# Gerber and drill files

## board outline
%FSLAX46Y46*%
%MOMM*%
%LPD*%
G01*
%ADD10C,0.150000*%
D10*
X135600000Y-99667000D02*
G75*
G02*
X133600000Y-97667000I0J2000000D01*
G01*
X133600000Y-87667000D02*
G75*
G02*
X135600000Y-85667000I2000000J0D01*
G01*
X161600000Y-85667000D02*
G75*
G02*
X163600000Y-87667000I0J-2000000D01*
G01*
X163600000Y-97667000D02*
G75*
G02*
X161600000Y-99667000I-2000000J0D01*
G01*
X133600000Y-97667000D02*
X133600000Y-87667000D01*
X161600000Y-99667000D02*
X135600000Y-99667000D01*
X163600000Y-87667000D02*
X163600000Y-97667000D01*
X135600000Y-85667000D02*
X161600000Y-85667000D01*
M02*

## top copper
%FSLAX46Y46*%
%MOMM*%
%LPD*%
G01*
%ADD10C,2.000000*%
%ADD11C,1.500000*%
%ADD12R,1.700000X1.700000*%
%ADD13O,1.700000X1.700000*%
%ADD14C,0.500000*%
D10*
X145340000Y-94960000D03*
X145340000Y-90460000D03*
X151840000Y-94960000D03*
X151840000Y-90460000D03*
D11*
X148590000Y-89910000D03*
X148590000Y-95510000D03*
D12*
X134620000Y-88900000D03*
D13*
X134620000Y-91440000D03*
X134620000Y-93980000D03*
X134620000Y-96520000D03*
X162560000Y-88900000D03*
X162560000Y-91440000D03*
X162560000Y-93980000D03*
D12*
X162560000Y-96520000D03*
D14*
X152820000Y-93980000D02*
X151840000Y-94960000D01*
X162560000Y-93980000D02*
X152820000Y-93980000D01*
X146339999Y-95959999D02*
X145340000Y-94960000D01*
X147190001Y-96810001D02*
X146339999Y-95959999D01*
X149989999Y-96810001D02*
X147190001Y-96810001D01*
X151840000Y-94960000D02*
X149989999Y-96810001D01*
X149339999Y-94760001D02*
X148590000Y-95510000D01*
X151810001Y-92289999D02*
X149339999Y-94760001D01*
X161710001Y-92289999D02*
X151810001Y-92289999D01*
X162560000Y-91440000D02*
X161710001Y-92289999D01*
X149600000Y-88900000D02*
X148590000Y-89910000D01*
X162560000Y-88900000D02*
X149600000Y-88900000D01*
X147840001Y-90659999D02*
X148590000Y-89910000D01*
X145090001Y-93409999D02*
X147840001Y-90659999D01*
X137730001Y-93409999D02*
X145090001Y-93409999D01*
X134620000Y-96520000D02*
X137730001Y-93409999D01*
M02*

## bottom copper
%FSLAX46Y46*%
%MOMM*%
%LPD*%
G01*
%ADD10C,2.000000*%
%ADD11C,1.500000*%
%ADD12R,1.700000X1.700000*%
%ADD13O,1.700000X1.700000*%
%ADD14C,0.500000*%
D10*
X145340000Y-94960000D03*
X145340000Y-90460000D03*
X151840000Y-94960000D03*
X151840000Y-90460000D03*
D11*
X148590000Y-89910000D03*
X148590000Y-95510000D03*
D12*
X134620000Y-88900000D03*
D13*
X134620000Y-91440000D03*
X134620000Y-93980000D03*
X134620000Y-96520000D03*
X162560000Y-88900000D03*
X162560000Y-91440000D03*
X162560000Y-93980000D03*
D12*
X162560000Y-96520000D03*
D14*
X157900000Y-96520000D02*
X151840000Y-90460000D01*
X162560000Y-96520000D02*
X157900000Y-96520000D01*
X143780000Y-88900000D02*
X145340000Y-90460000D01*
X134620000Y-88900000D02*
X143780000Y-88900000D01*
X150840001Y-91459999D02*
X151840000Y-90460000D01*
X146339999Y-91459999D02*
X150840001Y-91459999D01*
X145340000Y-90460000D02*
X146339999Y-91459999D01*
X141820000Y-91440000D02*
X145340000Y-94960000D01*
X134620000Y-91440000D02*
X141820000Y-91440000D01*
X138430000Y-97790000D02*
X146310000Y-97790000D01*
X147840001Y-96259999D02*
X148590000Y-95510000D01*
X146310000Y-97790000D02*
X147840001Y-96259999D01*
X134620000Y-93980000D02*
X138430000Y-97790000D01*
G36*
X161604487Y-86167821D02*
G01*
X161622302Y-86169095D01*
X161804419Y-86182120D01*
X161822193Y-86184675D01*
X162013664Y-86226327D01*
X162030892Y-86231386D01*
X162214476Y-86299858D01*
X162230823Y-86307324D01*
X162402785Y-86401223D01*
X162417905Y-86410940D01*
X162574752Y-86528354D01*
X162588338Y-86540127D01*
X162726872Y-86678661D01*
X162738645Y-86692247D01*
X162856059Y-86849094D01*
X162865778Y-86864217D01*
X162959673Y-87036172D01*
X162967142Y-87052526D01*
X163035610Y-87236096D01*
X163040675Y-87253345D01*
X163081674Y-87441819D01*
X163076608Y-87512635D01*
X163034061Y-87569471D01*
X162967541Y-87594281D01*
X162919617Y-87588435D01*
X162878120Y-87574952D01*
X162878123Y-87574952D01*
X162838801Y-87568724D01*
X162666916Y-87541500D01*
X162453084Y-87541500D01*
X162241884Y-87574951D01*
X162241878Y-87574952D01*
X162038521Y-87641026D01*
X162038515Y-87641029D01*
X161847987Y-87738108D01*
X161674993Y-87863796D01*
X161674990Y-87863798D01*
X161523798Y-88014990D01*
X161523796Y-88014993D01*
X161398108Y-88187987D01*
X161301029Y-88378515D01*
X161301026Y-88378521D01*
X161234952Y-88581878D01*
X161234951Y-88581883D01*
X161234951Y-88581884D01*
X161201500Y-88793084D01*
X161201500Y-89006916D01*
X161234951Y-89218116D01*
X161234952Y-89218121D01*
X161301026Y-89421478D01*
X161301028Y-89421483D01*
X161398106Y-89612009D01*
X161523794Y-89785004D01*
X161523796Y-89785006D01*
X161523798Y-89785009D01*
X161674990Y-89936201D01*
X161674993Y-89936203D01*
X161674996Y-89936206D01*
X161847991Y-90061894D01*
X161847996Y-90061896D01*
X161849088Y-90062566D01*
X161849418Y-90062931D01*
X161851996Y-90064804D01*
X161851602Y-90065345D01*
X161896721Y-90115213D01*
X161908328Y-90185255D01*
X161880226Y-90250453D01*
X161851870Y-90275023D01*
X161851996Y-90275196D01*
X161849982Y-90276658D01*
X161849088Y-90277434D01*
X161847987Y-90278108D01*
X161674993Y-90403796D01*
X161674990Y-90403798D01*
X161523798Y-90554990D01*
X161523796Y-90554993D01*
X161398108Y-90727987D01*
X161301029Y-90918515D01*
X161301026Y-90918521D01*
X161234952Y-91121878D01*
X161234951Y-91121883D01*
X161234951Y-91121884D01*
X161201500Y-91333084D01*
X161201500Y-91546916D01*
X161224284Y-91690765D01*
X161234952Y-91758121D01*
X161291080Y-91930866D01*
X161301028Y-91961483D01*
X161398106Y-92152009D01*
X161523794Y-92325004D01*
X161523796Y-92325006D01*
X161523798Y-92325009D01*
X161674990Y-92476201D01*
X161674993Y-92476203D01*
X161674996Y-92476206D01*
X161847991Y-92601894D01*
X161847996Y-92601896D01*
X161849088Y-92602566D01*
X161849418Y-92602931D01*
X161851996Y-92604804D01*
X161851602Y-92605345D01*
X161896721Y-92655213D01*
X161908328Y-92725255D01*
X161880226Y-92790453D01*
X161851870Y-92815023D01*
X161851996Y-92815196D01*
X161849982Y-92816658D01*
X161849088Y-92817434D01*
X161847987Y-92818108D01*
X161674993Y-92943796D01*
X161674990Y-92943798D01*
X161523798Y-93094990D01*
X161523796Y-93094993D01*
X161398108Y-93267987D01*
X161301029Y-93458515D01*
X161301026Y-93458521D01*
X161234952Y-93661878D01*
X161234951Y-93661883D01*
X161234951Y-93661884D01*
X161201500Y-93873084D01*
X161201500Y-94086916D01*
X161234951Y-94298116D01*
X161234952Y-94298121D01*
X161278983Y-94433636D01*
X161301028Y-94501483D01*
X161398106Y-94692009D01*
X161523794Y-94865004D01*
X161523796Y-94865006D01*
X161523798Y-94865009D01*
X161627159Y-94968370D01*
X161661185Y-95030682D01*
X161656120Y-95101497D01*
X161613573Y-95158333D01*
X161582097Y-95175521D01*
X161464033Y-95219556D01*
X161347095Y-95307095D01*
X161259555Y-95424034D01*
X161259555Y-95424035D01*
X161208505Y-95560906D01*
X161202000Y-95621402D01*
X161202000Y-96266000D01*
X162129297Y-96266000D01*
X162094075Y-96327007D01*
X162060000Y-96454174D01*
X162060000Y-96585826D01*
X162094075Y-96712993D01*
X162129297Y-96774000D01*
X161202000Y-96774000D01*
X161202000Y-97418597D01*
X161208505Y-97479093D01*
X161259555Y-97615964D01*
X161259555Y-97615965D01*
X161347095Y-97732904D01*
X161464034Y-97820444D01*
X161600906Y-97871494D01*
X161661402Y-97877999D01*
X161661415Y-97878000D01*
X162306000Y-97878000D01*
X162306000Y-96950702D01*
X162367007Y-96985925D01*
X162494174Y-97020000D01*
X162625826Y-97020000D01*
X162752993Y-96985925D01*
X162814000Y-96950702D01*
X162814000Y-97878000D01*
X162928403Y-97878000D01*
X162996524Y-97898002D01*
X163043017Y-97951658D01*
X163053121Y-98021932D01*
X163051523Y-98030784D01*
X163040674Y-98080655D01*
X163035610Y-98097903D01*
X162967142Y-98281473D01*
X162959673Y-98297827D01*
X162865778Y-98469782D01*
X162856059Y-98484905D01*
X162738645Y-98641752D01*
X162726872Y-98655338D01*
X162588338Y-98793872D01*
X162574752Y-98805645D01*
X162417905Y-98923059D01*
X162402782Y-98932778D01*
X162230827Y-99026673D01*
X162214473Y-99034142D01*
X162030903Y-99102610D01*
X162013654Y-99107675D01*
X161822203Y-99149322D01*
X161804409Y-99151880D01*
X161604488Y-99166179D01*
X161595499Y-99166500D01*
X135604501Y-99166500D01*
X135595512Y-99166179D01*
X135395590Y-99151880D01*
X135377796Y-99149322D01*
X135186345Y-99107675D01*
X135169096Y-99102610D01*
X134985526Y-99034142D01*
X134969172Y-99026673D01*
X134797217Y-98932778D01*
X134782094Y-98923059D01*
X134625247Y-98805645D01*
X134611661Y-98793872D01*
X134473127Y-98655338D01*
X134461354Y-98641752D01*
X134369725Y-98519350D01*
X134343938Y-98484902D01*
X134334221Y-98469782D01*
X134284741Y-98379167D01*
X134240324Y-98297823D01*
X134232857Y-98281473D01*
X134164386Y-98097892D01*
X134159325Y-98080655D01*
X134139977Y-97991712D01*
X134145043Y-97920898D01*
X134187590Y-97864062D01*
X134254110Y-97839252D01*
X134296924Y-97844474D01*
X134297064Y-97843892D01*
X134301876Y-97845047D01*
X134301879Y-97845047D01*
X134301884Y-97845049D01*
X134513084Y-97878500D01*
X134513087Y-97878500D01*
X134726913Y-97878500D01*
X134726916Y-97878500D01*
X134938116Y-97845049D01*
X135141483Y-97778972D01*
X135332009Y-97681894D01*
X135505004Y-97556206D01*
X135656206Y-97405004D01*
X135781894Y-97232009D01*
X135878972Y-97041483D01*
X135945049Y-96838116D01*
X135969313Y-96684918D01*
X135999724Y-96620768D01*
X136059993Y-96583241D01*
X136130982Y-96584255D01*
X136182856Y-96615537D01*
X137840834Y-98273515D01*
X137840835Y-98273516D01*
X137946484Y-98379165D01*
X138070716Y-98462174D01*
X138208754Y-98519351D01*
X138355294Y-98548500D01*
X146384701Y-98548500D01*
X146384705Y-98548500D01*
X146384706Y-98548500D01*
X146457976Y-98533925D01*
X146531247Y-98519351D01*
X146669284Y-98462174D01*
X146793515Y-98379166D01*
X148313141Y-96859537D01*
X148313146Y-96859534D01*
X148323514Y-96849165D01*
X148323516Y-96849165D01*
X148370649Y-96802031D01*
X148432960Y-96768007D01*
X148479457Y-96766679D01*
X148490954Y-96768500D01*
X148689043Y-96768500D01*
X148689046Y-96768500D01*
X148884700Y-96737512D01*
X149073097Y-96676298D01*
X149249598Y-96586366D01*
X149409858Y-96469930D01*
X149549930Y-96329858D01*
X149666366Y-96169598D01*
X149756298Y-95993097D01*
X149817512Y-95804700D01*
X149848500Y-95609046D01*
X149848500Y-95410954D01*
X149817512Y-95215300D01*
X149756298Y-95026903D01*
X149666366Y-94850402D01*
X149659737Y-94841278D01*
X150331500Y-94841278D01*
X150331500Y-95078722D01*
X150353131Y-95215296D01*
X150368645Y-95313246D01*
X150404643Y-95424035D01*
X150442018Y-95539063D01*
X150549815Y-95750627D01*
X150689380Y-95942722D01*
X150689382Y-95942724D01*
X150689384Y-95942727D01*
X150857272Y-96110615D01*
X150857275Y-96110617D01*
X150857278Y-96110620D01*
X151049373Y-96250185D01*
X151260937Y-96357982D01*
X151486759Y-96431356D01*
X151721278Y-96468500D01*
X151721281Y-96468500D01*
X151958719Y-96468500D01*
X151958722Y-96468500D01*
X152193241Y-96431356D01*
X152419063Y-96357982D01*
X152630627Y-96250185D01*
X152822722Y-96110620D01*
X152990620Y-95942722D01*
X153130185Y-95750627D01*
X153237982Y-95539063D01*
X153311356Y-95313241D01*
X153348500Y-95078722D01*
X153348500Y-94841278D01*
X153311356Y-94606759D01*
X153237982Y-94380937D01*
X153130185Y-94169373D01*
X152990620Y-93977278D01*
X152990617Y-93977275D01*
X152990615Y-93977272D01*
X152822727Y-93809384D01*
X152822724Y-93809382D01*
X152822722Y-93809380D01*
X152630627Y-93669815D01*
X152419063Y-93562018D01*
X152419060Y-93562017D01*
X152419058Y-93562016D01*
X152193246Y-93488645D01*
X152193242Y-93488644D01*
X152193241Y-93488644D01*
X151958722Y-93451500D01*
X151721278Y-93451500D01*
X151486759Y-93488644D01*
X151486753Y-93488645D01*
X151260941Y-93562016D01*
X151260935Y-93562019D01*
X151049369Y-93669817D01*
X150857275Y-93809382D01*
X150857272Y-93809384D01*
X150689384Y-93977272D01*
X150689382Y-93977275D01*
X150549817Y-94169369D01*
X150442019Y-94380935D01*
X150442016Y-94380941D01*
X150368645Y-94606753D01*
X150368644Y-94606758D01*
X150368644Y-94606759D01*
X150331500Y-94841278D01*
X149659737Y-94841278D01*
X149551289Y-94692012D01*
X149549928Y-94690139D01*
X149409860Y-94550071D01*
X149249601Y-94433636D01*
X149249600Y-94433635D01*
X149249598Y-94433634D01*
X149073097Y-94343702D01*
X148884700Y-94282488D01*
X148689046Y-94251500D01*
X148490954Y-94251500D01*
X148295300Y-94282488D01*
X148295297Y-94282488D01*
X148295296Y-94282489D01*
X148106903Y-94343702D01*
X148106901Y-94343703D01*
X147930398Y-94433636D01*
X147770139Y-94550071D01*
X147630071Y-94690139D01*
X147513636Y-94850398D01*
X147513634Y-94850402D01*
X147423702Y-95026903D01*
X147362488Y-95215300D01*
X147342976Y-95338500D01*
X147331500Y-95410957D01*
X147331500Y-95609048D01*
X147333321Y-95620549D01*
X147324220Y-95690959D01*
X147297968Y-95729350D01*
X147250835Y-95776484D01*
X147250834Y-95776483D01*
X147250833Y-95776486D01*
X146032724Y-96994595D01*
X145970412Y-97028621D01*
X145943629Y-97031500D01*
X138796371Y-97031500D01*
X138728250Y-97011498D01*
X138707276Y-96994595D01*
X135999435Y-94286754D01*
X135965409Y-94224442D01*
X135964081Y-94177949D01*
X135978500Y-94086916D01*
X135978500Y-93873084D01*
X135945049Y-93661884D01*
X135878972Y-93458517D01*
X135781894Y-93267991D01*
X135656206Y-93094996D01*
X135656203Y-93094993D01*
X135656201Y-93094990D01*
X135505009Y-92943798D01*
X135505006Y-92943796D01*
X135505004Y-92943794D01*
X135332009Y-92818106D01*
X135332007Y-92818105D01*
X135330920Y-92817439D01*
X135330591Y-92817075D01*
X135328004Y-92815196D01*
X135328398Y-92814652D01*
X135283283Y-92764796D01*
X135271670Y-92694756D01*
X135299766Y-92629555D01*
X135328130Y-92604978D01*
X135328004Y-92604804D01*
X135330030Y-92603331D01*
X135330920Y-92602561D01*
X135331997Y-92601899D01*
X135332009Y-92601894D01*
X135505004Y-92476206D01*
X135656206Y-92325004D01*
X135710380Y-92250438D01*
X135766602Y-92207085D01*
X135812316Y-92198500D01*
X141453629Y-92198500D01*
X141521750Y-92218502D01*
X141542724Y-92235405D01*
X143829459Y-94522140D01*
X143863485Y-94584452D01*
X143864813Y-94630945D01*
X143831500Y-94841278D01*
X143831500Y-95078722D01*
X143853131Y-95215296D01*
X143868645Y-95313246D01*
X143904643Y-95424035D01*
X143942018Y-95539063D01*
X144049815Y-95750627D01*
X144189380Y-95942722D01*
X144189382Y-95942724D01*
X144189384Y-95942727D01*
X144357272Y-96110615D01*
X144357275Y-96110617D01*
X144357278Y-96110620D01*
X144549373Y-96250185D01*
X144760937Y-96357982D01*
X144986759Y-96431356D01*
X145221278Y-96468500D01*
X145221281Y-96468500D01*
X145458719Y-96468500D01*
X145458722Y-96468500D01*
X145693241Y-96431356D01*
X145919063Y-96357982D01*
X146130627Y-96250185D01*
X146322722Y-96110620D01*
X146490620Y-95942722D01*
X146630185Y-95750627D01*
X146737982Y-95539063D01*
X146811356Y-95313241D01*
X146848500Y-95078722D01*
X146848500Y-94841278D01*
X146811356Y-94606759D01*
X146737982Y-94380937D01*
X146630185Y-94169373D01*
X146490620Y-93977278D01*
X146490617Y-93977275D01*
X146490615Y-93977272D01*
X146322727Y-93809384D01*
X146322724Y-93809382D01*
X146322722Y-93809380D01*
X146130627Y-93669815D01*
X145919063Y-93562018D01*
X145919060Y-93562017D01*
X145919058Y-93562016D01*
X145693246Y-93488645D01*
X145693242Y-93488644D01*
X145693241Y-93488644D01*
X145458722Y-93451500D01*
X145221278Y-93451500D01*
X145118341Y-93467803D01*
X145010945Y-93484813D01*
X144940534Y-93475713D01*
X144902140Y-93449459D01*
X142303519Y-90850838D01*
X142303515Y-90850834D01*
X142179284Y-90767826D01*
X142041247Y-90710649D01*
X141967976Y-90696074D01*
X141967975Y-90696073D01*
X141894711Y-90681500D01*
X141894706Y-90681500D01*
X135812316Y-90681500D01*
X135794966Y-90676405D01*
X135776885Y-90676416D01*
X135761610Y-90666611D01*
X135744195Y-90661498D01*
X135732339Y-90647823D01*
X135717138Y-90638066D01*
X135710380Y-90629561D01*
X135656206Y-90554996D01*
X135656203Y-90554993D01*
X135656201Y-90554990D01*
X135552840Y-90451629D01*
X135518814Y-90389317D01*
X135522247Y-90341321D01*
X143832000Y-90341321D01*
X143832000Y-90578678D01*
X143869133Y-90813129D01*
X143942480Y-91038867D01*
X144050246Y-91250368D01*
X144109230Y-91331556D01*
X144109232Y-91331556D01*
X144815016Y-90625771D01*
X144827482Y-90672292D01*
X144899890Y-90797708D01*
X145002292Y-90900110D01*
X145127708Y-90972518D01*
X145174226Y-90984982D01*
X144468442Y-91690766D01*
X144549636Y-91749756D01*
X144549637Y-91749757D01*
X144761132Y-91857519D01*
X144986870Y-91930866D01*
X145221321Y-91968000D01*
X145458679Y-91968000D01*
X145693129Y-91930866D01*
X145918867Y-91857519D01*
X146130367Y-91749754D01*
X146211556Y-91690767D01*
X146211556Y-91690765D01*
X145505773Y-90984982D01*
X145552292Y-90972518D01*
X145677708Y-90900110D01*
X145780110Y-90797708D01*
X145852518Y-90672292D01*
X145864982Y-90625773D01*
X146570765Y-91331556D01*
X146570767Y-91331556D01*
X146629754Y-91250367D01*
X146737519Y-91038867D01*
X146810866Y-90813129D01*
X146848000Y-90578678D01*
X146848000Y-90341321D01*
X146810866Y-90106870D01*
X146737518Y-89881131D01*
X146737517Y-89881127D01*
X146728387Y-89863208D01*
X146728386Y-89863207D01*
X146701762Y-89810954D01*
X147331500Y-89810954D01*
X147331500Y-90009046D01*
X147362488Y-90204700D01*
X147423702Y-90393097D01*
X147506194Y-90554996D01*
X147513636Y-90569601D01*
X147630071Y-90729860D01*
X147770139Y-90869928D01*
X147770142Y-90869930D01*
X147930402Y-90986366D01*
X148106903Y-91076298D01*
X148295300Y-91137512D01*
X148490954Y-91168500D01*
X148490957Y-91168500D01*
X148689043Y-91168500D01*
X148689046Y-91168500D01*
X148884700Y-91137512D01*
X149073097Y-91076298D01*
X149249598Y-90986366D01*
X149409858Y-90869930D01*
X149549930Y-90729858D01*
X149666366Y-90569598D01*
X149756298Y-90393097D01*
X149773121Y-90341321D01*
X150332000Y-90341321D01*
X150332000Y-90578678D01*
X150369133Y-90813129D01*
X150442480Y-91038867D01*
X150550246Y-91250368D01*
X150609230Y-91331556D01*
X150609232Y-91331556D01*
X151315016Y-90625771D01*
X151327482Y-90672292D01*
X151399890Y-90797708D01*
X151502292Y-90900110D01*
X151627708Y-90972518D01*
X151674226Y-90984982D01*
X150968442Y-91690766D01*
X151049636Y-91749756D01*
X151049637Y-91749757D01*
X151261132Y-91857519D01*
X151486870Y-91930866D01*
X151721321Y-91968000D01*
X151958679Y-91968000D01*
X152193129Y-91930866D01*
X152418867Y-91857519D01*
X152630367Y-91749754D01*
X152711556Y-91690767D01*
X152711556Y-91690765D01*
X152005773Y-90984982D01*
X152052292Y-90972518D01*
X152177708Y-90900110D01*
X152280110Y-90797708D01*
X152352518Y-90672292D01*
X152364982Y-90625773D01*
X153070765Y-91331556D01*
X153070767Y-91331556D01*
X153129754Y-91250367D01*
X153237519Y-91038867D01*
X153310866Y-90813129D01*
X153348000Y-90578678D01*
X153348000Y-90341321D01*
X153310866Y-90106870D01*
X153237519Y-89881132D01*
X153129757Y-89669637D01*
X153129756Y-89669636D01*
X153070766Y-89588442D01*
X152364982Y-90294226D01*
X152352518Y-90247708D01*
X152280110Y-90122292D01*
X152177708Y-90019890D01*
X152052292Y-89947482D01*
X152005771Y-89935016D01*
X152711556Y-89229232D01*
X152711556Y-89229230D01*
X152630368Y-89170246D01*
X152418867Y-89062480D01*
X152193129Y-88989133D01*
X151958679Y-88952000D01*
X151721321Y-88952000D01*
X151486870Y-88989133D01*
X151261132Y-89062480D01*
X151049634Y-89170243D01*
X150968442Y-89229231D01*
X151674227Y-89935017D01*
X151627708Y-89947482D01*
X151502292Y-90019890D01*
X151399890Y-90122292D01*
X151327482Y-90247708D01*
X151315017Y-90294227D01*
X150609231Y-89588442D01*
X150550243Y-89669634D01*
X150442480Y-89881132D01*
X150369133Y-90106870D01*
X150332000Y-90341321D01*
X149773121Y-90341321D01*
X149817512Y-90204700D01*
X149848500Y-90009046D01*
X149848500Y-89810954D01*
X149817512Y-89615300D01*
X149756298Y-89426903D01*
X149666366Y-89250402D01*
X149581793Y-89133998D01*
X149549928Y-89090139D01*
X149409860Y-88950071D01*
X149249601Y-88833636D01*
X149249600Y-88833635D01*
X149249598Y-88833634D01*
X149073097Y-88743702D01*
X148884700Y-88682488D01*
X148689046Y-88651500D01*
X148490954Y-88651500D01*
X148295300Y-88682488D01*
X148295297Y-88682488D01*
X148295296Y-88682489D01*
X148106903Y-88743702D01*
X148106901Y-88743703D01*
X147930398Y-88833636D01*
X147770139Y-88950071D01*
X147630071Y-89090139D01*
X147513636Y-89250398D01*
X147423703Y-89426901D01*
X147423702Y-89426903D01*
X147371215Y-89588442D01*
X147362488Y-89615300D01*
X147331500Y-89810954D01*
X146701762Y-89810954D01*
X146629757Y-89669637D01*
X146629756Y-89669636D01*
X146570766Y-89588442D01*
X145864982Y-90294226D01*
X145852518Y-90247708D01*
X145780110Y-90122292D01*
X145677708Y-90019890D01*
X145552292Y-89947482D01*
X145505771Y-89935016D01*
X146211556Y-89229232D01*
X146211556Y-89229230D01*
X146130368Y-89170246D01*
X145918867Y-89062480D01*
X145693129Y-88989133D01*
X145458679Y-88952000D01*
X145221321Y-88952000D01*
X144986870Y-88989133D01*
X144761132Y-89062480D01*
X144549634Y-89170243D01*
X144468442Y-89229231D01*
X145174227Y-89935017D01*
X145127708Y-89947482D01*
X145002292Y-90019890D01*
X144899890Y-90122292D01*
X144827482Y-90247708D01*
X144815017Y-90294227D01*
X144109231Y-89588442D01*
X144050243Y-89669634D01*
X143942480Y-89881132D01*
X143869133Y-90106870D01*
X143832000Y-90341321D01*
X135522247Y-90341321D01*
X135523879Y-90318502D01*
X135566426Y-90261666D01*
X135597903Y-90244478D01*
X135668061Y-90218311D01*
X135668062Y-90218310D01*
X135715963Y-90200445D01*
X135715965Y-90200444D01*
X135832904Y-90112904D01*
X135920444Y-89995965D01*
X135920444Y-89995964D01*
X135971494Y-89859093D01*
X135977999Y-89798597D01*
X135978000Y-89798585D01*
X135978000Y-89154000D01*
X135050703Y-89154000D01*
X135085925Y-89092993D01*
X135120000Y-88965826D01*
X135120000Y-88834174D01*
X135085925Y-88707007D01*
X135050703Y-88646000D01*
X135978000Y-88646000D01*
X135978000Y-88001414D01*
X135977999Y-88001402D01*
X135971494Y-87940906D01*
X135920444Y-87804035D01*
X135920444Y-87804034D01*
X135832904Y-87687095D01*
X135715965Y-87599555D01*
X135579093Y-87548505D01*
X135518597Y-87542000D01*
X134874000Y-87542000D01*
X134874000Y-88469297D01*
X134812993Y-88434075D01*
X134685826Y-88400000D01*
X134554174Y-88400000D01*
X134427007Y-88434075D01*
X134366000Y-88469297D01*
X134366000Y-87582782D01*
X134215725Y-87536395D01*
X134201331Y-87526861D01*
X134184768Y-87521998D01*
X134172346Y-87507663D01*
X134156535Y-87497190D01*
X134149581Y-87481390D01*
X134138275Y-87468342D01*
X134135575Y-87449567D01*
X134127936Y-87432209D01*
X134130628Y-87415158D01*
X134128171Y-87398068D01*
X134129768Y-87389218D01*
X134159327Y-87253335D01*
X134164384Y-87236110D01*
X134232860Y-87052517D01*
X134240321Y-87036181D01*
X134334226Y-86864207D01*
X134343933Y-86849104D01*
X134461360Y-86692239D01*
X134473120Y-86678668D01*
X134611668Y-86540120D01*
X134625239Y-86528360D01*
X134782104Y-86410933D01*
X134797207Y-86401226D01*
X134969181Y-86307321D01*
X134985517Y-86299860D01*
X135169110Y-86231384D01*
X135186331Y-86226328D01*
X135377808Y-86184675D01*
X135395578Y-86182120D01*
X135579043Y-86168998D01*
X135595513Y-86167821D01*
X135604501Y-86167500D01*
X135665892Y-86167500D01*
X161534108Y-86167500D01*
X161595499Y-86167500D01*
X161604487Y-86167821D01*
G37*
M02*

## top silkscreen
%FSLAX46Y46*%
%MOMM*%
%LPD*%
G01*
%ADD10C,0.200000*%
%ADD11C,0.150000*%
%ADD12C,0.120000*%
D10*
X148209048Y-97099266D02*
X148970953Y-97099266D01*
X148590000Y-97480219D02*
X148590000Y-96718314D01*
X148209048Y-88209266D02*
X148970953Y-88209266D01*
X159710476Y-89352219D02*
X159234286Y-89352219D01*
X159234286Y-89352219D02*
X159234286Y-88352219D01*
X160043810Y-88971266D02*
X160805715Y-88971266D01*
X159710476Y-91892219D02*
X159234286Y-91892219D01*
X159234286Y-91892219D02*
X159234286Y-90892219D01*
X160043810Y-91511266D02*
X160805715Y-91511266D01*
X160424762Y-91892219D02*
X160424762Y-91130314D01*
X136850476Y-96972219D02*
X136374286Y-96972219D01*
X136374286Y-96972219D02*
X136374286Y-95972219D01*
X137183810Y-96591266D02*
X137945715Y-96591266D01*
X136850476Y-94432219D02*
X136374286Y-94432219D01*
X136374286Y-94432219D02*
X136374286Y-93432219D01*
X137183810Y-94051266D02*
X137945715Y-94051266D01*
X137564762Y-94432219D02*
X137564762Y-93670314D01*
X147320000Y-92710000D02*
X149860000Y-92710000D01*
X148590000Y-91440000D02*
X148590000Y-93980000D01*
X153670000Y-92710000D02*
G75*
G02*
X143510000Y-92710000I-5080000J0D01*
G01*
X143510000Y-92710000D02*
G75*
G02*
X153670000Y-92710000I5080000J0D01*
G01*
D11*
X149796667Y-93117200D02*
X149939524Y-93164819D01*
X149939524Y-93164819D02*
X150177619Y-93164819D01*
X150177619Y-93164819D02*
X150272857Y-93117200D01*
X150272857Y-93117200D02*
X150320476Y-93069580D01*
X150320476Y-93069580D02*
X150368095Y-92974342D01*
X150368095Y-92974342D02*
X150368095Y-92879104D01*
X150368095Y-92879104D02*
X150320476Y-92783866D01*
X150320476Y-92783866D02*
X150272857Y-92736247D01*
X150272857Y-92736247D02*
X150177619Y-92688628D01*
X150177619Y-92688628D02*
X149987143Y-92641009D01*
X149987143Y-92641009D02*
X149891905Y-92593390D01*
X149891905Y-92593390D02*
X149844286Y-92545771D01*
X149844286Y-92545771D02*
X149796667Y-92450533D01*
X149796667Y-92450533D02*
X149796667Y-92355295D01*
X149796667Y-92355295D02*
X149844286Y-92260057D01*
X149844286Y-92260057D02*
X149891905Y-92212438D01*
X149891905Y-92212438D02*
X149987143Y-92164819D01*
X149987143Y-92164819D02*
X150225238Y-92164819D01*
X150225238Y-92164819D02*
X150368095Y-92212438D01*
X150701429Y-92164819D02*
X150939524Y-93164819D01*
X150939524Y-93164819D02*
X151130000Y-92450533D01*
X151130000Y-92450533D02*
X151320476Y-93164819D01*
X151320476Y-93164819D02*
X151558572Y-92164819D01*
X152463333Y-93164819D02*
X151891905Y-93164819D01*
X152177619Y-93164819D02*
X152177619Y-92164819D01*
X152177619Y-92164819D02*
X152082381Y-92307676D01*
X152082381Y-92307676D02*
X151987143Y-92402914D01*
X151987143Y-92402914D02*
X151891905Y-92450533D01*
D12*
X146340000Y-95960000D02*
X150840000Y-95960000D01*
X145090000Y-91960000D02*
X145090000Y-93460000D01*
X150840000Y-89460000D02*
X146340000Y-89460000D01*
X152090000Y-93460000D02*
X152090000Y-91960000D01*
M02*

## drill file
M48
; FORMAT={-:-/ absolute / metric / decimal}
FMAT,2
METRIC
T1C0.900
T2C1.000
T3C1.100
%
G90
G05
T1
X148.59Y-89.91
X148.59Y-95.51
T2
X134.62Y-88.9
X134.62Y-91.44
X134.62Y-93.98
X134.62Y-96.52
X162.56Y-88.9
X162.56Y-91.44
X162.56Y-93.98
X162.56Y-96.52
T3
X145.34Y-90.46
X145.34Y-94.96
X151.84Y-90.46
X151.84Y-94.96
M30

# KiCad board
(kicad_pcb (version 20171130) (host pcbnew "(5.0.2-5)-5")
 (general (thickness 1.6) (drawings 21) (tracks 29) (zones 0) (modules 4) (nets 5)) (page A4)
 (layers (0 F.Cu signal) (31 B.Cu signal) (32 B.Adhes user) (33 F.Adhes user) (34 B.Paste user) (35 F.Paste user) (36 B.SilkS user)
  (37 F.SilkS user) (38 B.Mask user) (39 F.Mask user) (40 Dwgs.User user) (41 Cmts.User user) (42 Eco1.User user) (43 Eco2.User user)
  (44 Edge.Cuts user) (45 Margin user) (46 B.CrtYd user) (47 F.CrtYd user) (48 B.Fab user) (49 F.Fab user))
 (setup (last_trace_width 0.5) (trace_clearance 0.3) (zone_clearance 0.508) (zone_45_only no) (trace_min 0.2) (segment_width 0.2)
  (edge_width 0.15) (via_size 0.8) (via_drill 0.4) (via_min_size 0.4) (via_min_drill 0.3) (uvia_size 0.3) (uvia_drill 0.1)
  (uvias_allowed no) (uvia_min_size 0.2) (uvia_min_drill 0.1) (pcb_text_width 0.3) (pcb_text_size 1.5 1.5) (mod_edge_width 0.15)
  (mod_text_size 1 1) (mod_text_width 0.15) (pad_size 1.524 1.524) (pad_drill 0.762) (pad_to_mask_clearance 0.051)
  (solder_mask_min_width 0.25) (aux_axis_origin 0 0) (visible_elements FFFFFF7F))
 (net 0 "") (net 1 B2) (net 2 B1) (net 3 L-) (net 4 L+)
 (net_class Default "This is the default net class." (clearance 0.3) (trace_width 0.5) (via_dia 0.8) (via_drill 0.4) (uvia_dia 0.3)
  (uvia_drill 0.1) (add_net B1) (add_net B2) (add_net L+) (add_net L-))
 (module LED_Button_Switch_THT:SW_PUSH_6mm (layer F.Cu) (at 145.34 90.46)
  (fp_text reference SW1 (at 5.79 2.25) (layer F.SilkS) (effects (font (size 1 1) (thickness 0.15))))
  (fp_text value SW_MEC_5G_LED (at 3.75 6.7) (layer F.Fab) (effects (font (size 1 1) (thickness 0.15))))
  (fp_line (start 1 5.5) (end 5.5 5.5) (layer F.SilkS) (width 0.12))
  (fp_line (start -0.25 1.5) (end -0.25 3) (layer F.SilkS) (width 0.12))
  (fp_line (start 5.5 -1) (end 1 -1) (layer F.SilkS) (width 0.12))
  (fp_line (start 6.75 3) (end 6.75 1.5) (layer F.SilkS) (width 0.12))
  (pad 4 thru_hole circle (at 0 4.5 90) (size 2 2) (drill 1.1) (layers *.Cu *.Mask) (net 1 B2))
  (pad 1 thru_hole circle (at 0 0 90) (size 2 2) (drill 1.1) (layers *.Cu *.Mask) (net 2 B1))
  (pad 4 thru_hole circle (at 6.5 4.5 90) (size 2 2) (drill 1.1) (layers *.Cu *.Mask) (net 1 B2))
  (pad 1 thru_hole circle (at 6.5 0 90) (size 2 2) (drill 1.1) (layers *.Cu *.Mask) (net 2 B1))
  (pad 2 thru_hole circle (at 3.25 -0.55 90) (size 1.5 1.5) (drill 0.9) (layers *.Cu *.Mask) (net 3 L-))
  (pad 3 thru_hole circle (at 3.25 5.05 90) (size 1.5 1.5) (drill 0.9) (layers *.Cu *.Mask) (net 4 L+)))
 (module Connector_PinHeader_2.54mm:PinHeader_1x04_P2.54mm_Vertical (layer B.Cu) (at 134.62 88.9 180)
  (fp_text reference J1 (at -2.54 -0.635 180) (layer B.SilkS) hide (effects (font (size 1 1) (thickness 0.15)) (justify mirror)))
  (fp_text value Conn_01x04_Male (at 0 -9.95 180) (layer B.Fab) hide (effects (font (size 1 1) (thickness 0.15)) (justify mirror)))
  (pad 1 thru_hole rect (at 0 0 180) (size 1.7 1.7) (drill 1) (layers *.Cu *.Mask) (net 2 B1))
  (pad 2 thru_hole oval (at 0 -2.54 180) (size 1.7 1.7) (drill 1) (layers *.Cu *.Mask) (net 1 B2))
  (pad 3 thru_hole oval (at 0 -5.08 180) (size 1.7 1.7) (drill 1) (layers *.Cu *.Mask) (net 4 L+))
  (pad 4 thru_hole oval (at 0 -7.62 180) (size 1.7 1.7) (drill 1) (layers *.Cu *.Mask) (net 3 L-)))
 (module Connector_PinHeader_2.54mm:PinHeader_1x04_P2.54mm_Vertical (layer B.Cu) (at 162.56 96.52)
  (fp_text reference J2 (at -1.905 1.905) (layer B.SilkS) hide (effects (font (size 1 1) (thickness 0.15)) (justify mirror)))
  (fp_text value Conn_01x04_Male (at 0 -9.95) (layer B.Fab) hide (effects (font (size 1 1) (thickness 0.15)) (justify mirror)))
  (pad 4 thru_hole oval (at 0 -7.62) (size 1.7 1.7) (drill 1) (layers *.Cu *.Mask) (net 3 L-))
  (pad 3 thru_hole oval (at 0 -5.08) (size 1.7 1.7) (drill 1) (layers *.Cu *.Mask) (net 4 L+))
  (pad 2 thru_hole oval (at 0 -2.54) (size 1.7 1.7) (drill 1) (layers *.Cu *.Mask) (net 1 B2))
  (pad 1 thru_hole rect (at 0 0) (size 1.7 1.7) (drill 1) (layers *.Cu *.Mask) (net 2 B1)))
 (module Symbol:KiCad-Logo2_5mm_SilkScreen (layer B.Cu) (at 156.845 92.71 90)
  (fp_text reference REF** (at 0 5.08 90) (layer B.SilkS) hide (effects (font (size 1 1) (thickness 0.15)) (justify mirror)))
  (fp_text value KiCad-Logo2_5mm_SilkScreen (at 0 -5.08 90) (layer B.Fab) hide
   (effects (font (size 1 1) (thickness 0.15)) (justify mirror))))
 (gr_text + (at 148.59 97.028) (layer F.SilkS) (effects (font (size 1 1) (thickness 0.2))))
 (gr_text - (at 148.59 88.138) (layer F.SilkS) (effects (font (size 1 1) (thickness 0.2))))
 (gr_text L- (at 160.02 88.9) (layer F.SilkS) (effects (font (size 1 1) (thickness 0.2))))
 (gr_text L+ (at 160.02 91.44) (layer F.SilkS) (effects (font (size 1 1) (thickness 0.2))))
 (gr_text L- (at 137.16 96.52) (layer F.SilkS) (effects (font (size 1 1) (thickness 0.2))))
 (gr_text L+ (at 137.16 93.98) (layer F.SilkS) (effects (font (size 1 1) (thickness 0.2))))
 (gr_line (start 147.32 92.71) (end 149.86 92.71) (layer F.SilkS) (width 0.2))
 (gr_line (start 148.59 91.44) (end 148.59 93.98) (layer F.SilkS) (width 0.2))
 (gr_circle (center 148.59 92.71) (end 153.67 92.71) (layer F.SilkS) (width 0.2))
 (gr_arc (start 135.6 97.667) (end 135.6 99.667) (angle 90) (layer Edge.Cuts) (width 0.15))
 (gr_arc (start 135.6 87.667) (end 133.6 87.667) (angle 90) (layer Edge.Cuts) (width 0.15))
 (gr_arc (start 161.6 87.667) (end 161.6 85.667) (angle 90) (layer Edge.Cuts) (width 0.15))
 (gr_arc (start 161.6 97.667) (end 163.6 97.667) (angle 90) (layer Edge.Cuts) (width 0.15))
 (gr_line (start 133.6 97.667) (end 133.6 87.667) (layer Edge.Cuts) (width 0.15))
 (gr_line (start 161.6 99.667) (end 135.6 99.667) (layer Edge.Cuts) (width 0.15))
 (gr_line (start 163.6 87.667) (end 163.6 97.667) (layer Edge.Cuts) (width 0.15))
 (gr_line (start 135.6 85.667) (end 161.6 85.667) (layer Edge.Cuts) (width 0.15))
 (segment (start 157.9 96.52) (end 151.84 90.46) (width 0.5) (layer B.Cu) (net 2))
 (segment (start 162.56 96.52) (end 157.9 96.52) (width 0.5) (layer B.Cu) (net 2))
 (segment (start 143.78 88.9) (end 145.34 90.46) (width 0.5) (layer B.Cu) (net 2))
 (segment (start 134.62 88.9) (end 143.78 88.9) (width 0.5) (layer B.Cu) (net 2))
 (segment (start 150.840001 91.459999) (end 151.84 90.46) (width 0.5) (layer B.Cu) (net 2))
 (segment (start 146.339999 91.459999) (end 150.840001 91.459999) (width 0.5) (layer B.Cu) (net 2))
 (segment (start 145.34 90.46) (end 146.339999 91.459999) (width 0.5) (layer B.Cu) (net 2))
 (segment (start 152.82 93.98) (end 151.84 94.96) (width 0.5) (layer F.Cu) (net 1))
 (segment (start 162.56 93.98) (end 152.82 93.98) (width 0.5) (layer F.Cu) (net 1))
 (segment (start 146.339999 95.959999) (end 145.34 94.96) (width 0.5) (layer F.Cu) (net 1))
 (segment (start 147.190001 96.810001) (end 146.339999 95.959999) (width 0.5) (layer F.Cu) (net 1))
 (segment (start 149.989999 96.810001) (end 147.190001 96.810001) (width 0.5) (layer F.Cu) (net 1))
 (segment (start 151.84 94.96) (end 149.989999 96.810001) (width 0.5) (layer F.Cu) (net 1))
 (segment (start 141.82 91.44) (end 145.34 94.96) (width 0.5) (layer B.Cu) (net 1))
 (segment (start 134.62 91.44) (end 141.82 91.44) (width 0.5) (layer B.Cu) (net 1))
 (segment (start 149.339999 94.760001) (end 148.59 95.51) (width 0.5) (layer F.Cu) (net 4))
 (segment (start 151.810001 92.289999) (end 149.339999 94.760001) (width 0.5) (layer F.Cu) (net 4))
 (segment (start 161.710001 92.289999) (end 151.810001 92.289999) (width 0.5) (layer F.Cu) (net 4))
 (segment (start 162.56 91.44) (end 161.710001 92.289999) (width 0.5) (layer F.Cu) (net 4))
 (segment (start 138.43 97.79) (end 146.31 97.79) (width 0.5) (layer B.Cu) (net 4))
 (segment (start 147.840001 96.259999) (end 148.59 95.51) (width 0.5) (layer B.Cu) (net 4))
 (segment (start 146.31 97.79) (end 147.840001 96.259999) (width 0.5) (layer B.Cu) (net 4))
 (segment (start 134.62 93.98) (end 138.43 97.79) (width 0.5) (layer B.Cu) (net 4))
 (segment (start 149.6 88.9) (end 148.59 89.91) (width 0.5) (layer F.Cu) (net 3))
 (segment (start 162.56 88.9) (end 149.6 88.9) (width 0.5) (layer F.Cu) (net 3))
 (segment (start 147.840001 90.659999) (end 148.59 89.91) (width 0.5) (layer F.Cu) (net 3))
 (segment (start 145.090001 93.409999) (end 147.840001 90.659999) (width 0.5) (layer F.Cu) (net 3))
 (segment (start 137.730001 93.409999) (end 145.090001 93.409999) (width 0.5) (layer F.Cu) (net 3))
 (segment (start 134.62 96.52) (end 137.730001 93.409999) (width 0.5) (layer F.Cu) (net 3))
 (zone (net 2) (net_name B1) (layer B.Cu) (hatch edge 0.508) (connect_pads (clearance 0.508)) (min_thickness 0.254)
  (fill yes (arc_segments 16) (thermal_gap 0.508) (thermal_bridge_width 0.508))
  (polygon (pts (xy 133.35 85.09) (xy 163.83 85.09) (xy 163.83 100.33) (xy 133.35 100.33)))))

